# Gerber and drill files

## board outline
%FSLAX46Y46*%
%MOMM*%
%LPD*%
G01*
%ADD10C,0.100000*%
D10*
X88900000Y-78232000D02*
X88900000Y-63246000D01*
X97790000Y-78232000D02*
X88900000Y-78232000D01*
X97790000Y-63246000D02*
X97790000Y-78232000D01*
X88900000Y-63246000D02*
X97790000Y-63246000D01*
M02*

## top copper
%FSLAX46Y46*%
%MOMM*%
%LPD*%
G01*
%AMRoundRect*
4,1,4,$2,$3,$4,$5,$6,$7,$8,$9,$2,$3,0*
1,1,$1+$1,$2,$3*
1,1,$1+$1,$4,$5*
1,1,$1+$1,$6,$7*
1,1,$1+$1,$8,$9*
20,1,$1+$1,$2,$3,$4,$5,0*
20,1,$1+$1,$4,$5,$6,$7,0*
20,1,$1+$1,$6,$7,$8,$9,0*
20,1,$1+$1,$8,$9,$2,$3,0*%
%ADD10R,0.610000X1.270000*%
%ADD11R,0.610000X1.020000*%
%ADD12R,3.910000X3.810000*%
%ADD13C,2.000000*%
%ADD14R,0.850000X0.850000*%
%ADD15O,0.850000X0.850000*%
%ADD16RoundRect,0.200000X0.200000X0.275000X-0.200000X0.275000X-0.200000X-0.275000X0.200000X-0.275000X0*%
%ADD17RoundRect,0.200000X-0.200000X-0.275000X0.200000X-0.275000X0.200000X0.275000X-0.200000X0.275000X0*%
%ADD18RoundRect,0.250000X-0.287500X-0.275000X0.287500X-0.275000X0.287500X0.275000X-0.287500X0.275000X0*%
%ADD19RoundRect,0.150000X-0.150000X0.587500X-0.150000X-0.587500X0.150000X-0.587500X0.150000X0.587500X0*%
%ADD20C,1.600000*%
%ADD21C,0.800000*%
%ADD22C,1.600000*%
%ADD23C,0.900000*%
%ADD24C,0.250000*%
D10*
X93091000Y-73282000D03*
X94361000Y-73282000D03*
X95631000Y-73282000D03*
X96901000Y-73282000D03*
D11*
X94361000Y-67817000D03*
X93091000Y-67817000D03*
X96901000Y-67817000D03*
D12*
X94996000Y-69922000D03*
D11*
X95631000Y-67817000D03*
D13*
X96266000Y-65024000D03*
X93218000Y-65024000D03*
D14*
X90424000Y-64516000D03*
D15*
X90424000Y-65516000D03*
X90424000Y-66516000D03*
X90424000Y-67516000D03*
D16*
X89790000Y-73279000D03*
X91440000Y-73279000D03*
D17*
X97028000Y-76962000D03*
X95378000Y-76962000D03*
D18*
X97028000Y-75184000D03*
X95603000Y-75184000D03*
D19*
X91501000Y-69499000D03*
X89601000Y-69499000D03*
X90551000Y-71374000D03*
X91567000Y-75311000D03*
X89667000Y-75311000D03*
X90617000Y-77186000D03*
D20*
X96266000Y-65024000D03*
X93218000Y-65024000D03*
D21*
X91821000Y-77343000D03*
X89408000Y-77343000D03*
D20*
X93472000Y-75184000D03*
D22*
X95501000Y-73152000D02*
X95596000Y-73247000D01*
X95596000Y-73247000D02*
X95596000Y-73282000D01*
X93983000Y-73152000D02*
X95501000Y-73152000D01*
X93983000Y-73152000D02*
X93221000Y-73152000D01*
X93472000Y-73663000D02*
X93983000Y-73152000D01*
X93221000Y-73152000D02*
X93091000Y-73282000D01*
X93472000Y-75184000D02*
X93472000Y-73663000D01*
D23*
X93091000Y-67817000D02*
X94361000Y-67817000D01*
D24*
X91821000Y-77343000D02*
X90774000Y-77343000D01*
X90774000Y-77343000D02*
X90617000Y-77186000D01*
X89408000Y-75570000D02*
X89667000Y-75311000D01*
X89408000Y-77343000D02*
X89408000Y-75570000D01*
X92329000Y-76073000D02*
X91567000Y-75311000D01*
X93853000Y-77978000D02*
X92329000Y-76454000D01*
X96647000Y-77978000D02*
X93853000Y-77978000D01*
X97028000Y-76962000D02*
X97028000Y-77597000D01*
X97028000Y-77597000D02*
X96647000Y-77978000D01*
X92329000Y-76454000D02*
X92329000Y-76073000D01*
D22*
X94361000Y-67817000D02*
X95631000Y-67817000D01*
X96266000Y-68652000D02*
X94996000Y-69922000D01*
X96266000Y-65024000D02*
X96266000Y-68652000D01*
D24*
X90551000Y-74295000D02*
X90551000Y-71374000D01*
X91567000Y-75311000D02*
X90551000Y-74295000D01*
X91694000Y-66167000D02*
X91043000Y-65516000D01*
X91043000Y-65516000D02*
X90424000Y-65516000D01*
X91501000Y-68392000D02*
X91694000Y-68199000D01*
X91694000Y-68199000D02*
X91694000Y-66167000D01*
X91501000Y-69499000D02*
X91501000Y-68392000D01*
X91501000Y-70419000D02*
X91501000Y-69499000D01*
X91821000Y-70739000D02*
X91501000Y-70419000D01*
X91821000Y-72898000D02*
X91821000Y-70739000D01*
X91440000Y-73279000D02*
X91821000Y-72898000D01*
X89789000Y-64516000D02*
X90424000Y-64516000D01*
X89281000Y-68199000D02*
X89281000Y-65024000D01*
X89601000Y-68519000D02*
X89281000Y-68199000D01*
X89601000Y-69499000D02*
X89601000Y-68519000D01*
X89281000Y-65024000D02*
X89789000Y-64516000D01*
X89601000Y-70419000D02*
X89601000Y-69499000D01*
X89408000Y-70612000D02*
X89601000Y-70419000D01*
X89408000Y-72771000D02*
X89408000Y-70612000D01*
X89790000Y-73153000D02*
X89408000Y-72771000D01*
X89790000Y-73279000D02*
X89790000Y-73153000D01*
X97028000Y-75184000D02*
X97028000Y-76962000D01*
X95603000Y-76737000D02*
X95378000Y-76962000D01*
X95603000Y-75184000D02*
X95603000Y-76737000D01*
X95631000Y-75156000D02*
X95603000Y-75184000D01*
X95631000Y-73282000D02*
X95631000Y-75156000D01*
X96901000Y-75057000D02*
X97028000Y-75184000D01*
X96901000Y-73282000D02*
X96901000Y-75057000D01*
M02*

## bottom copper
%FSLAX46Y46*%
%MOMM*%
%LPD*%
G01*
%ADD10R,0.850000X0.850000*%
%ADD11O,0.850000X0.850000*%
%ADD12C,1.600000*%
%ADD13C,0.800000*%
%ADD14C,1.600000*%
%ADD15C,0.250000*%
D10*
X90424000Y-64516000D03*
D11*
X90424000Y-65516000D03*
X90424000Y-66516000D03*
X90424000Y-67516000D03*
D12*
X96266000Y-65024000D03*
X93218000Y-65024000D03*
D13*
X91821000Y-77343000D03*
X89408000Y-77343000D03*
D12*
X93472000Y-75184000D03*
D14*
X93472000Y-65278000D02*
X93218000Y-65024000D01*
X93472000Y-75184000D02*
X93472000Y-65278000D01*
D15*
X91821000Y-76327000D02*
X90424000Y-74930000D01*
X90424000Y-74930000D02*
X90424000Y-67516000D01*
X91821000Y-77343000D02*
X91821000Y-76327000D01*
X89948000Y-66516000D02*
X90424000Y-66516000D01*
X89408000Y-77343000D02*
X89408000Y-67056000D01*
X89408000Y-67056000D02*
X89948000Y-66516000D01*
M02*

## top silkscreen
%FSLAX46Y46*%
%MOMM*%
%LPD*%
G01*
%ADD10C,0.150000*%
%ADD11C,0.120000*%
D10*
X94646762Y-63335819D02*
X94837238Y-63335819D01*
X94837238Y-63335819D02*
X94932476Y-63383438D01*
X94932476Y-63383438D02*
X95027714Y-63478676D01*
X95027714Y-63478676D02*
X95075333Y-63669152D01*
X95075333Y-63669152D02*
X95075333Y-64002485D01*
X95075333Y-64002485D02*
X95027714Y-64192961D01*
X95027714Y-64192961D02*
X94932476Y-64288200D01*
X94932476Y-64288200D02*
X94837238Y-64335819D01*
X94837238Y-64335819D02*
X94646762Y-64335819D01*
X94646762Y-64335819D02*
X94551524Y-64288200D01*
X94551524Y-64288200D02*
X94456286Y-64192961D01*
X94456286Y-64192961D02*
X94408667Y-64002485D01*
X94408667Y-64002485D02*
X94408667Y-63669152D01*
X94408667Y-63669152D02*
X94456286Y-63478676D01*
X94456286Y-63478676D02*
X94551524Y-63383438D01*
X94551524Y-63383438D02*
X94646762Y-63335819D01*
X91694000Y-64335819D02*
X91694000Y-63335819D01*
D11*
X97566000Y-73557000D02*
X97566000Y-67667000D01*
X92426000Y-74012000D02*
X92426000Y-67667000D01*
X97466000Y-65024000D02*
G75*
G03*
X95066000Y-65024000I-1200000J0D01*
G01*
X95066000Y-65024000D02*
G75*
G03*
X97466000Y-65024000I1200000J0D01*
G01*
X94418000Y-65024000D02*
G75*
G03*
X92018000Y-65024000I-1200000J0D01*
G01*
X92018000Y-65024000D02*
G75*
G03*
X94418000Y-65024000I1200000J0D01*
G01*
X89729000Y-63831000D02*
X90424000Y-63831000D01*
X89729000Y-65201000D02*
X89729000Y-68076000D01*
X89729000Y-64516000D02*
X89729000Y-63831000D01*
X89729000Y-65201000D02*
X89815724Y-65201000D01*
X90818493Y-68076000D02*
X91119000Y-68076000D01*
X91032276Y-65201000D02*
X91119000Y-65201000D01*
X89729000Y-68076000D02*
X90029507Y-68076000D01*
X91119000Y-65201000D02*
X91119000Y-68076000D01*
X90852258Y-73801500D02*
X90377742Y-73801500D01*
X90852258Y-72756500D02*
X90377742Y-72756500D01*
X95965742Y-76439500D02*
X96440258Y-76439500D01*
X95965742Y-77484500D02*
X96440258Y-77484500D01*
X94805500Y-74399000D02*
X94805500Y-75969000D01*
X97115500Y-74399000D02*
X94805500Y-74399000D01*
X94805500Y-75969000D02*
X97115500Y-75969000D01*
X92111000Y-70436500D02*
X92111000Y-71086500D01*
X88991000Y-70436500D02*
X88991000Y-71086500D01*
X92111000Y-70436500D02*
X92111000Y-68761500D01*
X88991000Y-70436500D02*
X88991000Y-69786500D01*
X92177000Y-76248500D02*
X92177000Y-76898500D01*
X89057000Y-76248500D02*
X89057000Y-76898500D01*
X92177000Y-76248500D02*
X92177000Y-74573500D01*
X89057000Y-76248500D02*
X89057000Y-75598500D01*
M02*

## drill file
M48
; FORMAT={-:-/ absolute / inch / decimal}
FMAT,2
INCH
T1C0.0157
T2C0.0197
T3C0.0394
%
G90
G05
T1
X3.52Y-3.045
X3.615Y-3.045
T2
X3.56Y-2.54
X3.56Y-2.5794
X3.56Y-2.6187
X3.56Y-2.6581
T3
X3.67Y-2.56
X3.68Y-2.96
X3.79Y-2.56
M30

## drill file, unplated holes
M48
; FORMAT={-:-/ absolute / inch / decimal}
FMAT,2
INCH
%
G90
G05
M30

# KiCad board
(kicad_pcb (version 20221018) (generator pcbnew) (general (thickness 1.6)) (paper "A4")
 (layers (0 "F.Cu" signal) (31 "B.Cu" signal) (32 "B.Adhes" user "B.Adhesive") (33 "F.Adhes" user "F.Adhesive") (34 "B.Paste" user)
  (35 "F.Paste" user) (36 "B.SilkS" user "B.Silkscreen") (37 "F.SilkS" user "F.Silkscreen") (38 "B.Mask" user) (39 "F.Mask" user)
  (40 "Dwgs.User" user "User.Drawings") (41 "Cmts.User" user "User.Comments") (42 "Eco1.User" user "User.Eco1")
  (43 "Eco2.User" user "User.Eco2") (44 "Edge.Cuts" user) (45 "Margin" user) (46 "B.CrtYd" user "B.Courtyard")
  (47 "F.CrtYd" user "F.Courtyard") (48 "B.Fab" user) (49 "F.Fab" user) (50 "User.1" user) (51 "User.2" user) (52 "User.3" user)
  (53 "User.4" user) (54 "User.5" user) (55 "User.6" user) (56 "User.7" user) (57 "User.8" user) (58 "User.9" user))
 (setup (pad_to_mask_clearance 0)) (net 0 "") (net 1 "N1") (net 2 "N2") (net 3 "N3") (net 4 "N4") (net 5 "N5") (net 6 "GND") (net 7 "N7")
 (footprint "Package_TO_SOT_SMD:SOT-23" (layer "F.Cu") (at 90.617 76.2485 -90)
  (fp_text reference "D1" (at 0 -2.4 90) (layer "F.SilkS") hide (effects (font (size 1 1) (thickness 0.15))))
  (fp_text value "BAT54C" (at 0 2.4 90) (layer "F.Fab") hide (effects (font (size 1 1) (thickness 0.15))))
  (fp_line (start 0 -1.56) (end -1.675 -1.56) (stroke (width 0.12) (type solid)) (layer "F.SilkS"))
  (fp_line (start 0 -1.56) (end 0.65 -1.56) (stroke (width 0.12) (type solid)) (layer "F.SilkS"))
  (fp_line (start 0 1.56) (end -0.65 1.56) (stroke (width 0.12) (type solid)) (layer "F.SilkS"))
  (fp_line (start 0 1.56) (end 0.65 1.56) (stroke (width 0.12) (type solid)) (layer "F.SilkS"))
  (pad "1" smd roundrect (at -0.9375 -0.95 270) (size 1.475 0.6) (layers "F.Cu" "F.Paste" "F.Mask") (roundrect_rratio 0.25) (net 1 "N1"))
  (pad "2" smd roundrect (at -0.9375 0.95 270) (size 1.475 0.6) (layers "F.Cu" "F.Paste" "F.Mask") (roundrect_rratio 0.25) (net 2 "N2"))
  (pad "3" smd roundrect (at 0.9375 0 270) (size 1.475 0.6) (layers "F.Cu" "F.Paste" "F.Mask") (roundrect_rratio 0.25) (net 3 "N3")))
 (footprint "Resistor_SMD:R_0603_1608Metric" (layer "F.Cu") (at 96.203 76.962)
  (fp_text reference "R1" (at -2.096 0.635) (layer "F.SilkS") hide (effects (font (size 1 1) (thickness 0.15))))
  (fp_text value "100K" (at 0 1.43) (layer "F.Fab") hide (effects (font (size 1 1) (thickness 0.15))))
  (fp_line (start -0.237258 -0.5225) (end 0.237258 -0.5225) (stroke (width 0.12) (type solid)) (layer "F.SilkS"))
  (fp_line (start -0.237258 0.5225) (end 0.237258 0.5225) (stroke (width 0.12) (type solid)) (layer "F.SilkS"))
  (pad "1" smd roundrect (at -0.825 0) (size 0.8 0.95) (layers "F.Cu" "F.Paste" "F.Mask") (roundrect_rratio 0.25) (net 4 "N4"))
  (pad "2" smd roundrect (at 0.825 0) (size 0.8 0.95) (layers "F.Cu" "F.Paste" "F.Mask") (roundrect_rratio 0.25) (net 1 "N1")))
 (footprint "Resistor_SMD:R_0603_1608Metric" (layer "F.Cu") (at 90.615 73.279 180)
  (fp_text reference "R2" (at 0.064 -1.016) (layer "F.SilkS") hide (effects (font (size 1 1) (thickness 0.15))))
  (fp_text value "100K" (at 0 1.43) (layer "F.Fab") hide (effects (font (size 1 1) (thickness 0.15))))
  (fp_line (start -0.237258 -0.5225) (end 0.237258 -0.5225) (stroke (width 0.12) (type solid)) (layer "F.SilkS"))
  (fp_line (start -0.237258 0.5225) (end 0.237258 0.5225) (stroke (width 0.12) (type solid)) (layer "F.SilkS"))
  (pad "1" smd roundrect (at -0.825 0 180) (size 0.8 0.95) (layers "F.Cu" "F.Paste" "F.Mask") (roundrect_rratio 0.25) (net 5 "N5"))
  (pad "2" smd roundrect (at 0.825 0 180) (size 0.8 0.95) (layers "F.Cu" "F.Paste" "F.Mask") (roundrect_rratio 0.25) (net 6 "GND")))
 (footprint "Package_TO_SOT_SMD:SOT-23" (layer "F.Cu") (at 90.551 70.4365 -90)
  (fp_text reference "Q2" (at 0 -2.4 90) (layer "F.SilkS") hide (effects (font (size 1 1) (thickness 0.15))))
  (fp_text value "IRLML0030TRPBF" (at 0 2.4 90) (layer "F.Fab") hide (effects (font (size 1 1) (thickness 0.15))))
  (fp_line (start 0 -1.56) (end -1.675 -1.56) (stroke (width 0.12) (type solid)) (layer "F.SilkS"))
  (fp_line (start 0 -1.56) (end 0.65 -1.56) (stroke (width 0.12) (type solid)) (layer "F.SilkS"))
  (fp_line (start 0 1.56) (end -0.65 1.56) (stroke (width 0.12) (type solid)) (layer "F.SilkS"))
  (fp_line (start 0 1.56) (end 0.65 1.56) (stroke (width 0.12) (type solid)) (layer "F.SilkS"))
  (pad "1" smd roundrect (at -0.9375 -0.95 270) (size 1.475 0.6) (layers "F.Cu" "F.Paste" "F.Mask") (roundrect_rratio 0.25) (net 5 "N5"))
  (pad "2" smd roundrect (at -0.9375 0.95 270) (size 1.475 0.6) (layers "F.Cu" "F.Paste" "F.Mask") (roundrect_rratio 0.25) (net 6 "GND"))
  (pad "3" smd roundrect (at 0.9375 0 270) (size 1.475 0.6) (layers "F.Cu" "F.Paste" "F.Mask") (roundrect_rratio 0.25) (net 1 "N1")))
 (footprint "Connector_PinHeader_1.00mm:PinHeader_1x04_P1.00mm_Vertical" (layer "F.Cu") (at 90.424 64.516)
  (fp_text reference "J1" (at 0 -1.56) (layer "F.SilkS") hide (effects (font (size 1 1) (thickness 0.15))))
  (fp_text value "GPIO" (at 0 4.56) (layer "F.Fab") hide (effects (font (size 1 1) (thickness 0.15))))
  (fp_line (start -0.695 -0.685) (end 0 -0.685) (stroke (width 0.12) (type solid)) (layer "F.SilkS"))
  (fp_line (start -0.695 0) (end -0.695 -0.685) (stroke (width 0.12) (type solid)) (layer "F.SilkS"))
  (fp_line (start -0.695 0.685) (end -0.695 3.56) (stroke (width 0.12) (type solid)) (layer "F.SilkS"))
  (fp_line (start -0.695 0.685) (end -0.608276 0.685) (stroke (width 0.12) (type solid)) (layer "F.SilkS"))
  (fp_line (start -0.695 3.56) (end -0.394493 3.56) (stroke (width 0.12) (type solid)) (layer "F.SilkS"))
  (fp_line (start 0.394493 3.56) (end 0.695 3.56) (stroke (width 0.12) (type solid)) (layer "F.SilkS"))
  (fp_line (start 0.608276 0.685) (end 0.695 0.685) (stroke (width 0.12) (type solid)) (layer "F.SilkS"))
  (fp_line (start 0.695 0.685) (end 0.695 3.56) (stroke (width 0.12) (type solid)) (layer "F.SilkS"))
  (pad "1" thru_hole rect (at 0 0) (size 0.85 0.85) (drill 0.5) (layers "*.Cu" "*.Mask") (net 6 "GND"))
  (pad "2" thru_hole oval (at 0 1) (size 0.85 0.85) (drill 0.5) (layers "*.Cu" "*.Mask") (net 5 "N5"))
  (pad "3" thru_hole oval (at 0 2) (size 0.85 0.85) (drill 0.5) (layers "*.Cu" "*.Mask") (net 2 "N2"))
  (pad "4" thru_hole oval (at 0 3) (size 0.85 0.85) (drill 0.5) (layers "*.Cu" "*.Mask") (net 3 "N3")))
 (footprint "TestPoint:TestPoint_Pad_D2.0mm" (layer "F.Cu") (at 96.266 65.024)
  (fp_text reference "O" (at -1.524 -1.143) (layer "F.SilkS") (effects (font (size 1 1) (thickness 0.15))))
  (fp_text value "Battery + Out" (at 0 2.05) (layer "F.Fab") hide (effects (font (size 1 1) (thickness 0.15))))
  (fp_circle (center 0 0) (end 0 1.2) (stroke (width 0.12) (type solid)) (fill none) (layer "F.SilkS"))
  (pad "1" smd circle (at 0 0) (size 2 2) (layers "F.Cu" "F.Mask") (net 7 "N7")))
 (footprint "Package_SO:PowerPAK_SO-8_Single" (layer "F.Cu") (at 94.996 70.612 90)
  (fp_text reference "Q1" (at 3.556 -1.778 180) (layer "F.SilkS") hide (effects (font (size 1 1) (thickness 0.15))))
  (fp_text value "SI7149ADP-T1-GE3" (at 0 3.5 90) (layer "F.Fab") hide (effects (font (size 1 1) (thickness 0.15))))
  (fp_line (start -3.4 -2.57) (end 2.945 -2.57) (stroke (width 0.12) (type solid)) (layer "F.SilkS"))
  (fp_line (start -2.945 2.57) (end 2.945 2.57) (stroke (width 0.12) (type solid)) (layer "F.SilkS"))
  (pad "1" smd rect (at -2.67 -1.905 90) (size 1.27 0.61) (layers "F.Cu" "F.Paste" "F.Mask") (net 4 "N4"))
  (pad "2" smd rect (at -2.67 -0.635 90) (size 1.27 0.61) (layers "F.Cu" "F.Paste" "F.Mask") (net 4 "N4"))
  (pad "3" smd rect (at -2.67 0.635 90) (size 1.27 0.61) (layers "F.Cu" "F.Paste" "F.Mask") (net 4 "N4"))
  (pad "4" smd rect (at -2.67 1.905 90) (size 1.27 0.61) (layers "F.Cu" "F.Paste" "F.Mask") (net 1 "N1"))
  (pad "5" smd rect (at 0.69 0 90) (size 3.81 3.91) (layers "F.Cu" "F.Paste" "F.Mask") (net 7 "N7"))
  (pad "5" smd rect (at 2.795 -1.905 90) (size 1.02 0.61) (layers "F.Cu" "F.Paste" "F.Mask") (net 7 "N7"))
  (pad "5" smd rect (at 2.795 -0.635 90) (size 1.02 0.61) (layers "F.Cu" "F.Paste" "F.Mask") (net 7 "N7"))
  (pad "5" smd rect (at 2.795 0.635 90) (size 1.02 0.61) (layers "F.Cu" "F.Paste" "F.Mask") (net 7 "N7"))
  (pad "5" smd rect (at 2.795 1.905 90) (size 1.02 0.61) (layers "F.Cu" "F.Paste" "F.Mask") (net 7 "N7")))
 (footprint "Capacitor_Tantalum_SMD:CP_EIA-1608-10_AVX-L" (layer "F.Cu") (at 96.3155 75.184)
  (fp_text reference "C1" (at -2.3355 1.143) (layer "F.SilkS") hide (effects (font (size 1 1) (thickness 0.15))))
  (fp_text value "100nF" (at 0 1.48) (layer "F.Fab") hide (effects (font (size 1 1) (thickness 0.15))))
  (fp_line (start -1.51 -0.785) (end -1.51 0.785) (stroke (width 0.12) (type solid)) (layer "F.SilkS"))
  (fp_line (start -1.51 0.785) (end 0.8 0.785) (stroke (width 0.12) (type solid)) (layer "F.SilkS"))
  (fp_line (start 0.8 -0.785) (end -1.51 -0.785) (stroke (width 0.12) (type solid)) (layer "F.SilkS"))
  (pad "1" smd roundrect (at -0.7125 0) (size 1.075 1.05) (layers "F.Cu" "F.Paste" "F.Mask") (roundrect_rratio 0.2380952381) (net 4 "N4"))
  (pad "2" smd roundrect (at 0.7125 0) (size 1.075 1.05) (layers "F.Cu" "F.Paste" "F.Mask") (roundrect_rratio 0.2380952381) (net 1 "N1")))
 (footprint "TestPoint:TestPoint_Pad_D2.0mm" (layer "F.Cu") (at 93.218 65.024)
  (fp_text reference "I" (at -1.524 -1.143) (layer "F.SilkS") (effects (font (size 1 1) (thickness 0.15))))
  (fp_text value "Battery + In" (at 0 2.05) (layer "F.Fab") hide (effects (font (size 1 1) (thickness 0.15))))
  (fp_circle (center 0 0) (end 0 1.2) (stroke (width 0.12) (type solid)) (fill none) (layer "F.SilkS"))
  (pad "1" smd circle (at 0 0) (size 2 2) (layers "F.Cu" "F.Mask") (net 4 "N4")))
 (gr_line (start 97.79 63.246) (end 97.79 78.232) (stroke (width 0.1) (type default)) (layer "Edge.Cuts"))
 (gr_line (start 88.9 63.246) (end 97.79 63.246) (stroke (width 0.1) (type default)) (layer "Edge.Cuts"))
 (gr_line (start 88.9 78.232) (end 88.9 63.246) (stroke (width 0.1) (type default)) (layer "Edge.Cuts"))
 (gr_line (start 97.79 78.232) (end 88.9 78.232) (stroke (width 0.1) (type default)) (layer "Edge.Cuts"))
 (segment (start 91.501 70.419) (end 91.501 69.499) (width 0.25) (layer "F.Cu") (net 5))
 (segment (start 91.694 68.199) (end 91.694 66.167) (width 0.25) (layer "F.Cu") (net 5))
 (segment (start 91.043 65.516) (end 90.424 65.516) (width 0.25) (layer "F.Cu") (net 5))
 (segment (start 91.501 68.392) (end 91.694 68.199) (width 0.25) (layer "F.Cu") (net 5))
 (segment (start 91.694 66.167) (end 91.043 65.516) (width 0.25) (layer "F.Cu") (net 5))
 (segment (start 91.44 73.279) (end 91.821 72.898) (width 0.25) (layer "F.Cu") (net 5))
 (segment (start 91.821 70.739) (end 91.501 70.419) (width 0.25) (layer "F.Cu") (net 5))
 (segment (start 91.821 72.898) (end 91.821 70.739) (width 0.25) (layer "F.Cu") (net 5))
 (segment (start 91.501 69.499) (end 91.501 68.392) (width 0.25) (layer "F.Cu") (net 5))
 (segment (start 89.408 77.343) (end 89.408 75.57) (width 0.25) (layer "F.Cu") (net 2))
 (segment (start 89.408 75.57) (end 89.667 75.311) (width 0.25) (layer "F.Cu") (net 2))
 (via (at 89.408 77.343) (size 0.8) (drill 0.4) (layers "F.Cu" "B.Cu") (free) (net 2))
 (segment (start 89.408 77.343) (end 89.408 67.056) (width 0.25) (layer "B.Cu") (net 2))
 (segment (start 89.408 67.056) (end 89.948 66.516) (width 0.25) (layer "B.Cu") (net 2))
 (segment (start 89.948 66.516) (end 90.424 66.516) (width 0.25) (layer "B.Cu") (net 2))
 (segment (start 97.028 75.184) (end 97.028 76.962) (width 0.25) (layer "F.Cu") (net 1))
 (segment (start 92.329 76.073) (end 91.567 75.311) (width 0.25) (layer "F.Cu") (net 1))
 (segment (start 97.028 76.962) (end 97.028 77.597) (width 0.25) (layer "F.Cu") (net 1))
 (segment (start 91.567 75.311) (end 90.551 74.295) (width 0.25) (layer "F.Cu") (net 1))
 (segment (start 96.901 75.057) (end 97.028 75.184) (width 0.25) (layer "F.Cu") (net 1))
 (segment (start 96.901 73.282) (end 96.901 75.057) (width 0.25) (layer "F.Cu") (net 1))
 (segment (start 92.329 76.454) (end 92.329 76.073) (width 0.25) (layer "F.Cu") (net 1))
 (segment (start 96.647 77.978) (end 93.853 77.978) (width 0.25) (layer "F.Cu") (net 1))
 (segment (start 90.551 74.295) (end 90.551 71.374) (width 0.25) (layer "F.Cu") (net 1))
 (segment (start 93.853 77.978) (end 92.329 76.454) (width 0.25) (layer "F.Cu") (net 1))
 (segment (start 97.028 77.597) (end 96.647 77.978) (width 0.25) (layer "F.Cu") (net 1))
 (segment (start 93.472 73.663) (end 93.983 73.152) (width 1.6) (layer "F.Cu") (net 4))
 (segment (start 95.603 76.737) (end 95.378 76.962) (width 0.25) (layer "F.Cu") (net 4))
 (segment (start 95.596 73.247) (end 95.596 73.282) (width 1.6) (layer "F.Cu") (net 4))
 (segment (start 93.221 73.152) (end 93.091 73.282) (width 1.6) (layer "F.Cu") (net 4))
 (segment (start 95.603 75.184) (end 95.603 76.737) (width 0.25) (layer "F.Cu") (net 4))
 (segment (start 93.983 73.152) (end 95.501 73.152) (width 1.6) (layer "F.Cu") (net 4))
 (segment (start 95.501 73.152) (end 95.596 73.247) (width 1.6) (layer "F.Cu") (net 4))
 (segment (start 93.472 75.184) (end 93.472 73.663) (width 1.6) (layer "F.Cu") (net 4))
 (segment (start 95.631 75.156) (end 95.603 75.184) (width 0.25) (layer "F.Cu") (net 4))
 (segment (start 95.631 73.282) (end 95.631 75.156) (width 0.25) (layer "F.Cu") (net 4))
 (segment (start 93.983 73.152) (end 93.221 73.152) (width 1.6) (layer "F.Cu") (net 4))
 (via (at 93.218 65.024) (size 1.6) (drill 1) (layers "F.Cu" "B.Cu") (free) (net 4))
 (via (at 93.472 75.184) (size 1.6) (drill 1) (layers "F.Cu" "B.Cu") (free) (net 4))
 (segment (start 93.472 75.184) (end 93.472 65.278) (width 1.6) (layer "B.Cu") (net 4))
 (segment (start 93.472 65.278) (end 93.218 65.024) (width 1.6) (layer "B.Cu") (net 4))
 (segment (start 96.266 68.652) (end 94.996 69.922) (width 1.6) (layer "F.Cu") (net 7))
 (segment (start 93.091 67.817) (end 94.361 67.817) (width 0.9) (layer "F.Cu") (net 7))
 (segment (start 94.361 67.817) (end 95.631 67.817) (width 1.6) (layer "F.Cu") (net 7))
 (segment (start 96.266 65.024) (end 96.266 68.652) (width 1.6) (layer "F.Cu") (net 7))
 (via (at 96.266 65.024) (size 1.6) (drill 1) (layers "F.Cu" "B.Cu") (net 7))
 (segment (start 89.79 73.153) (end 89.408 72.771) (width 0.25) (layer "F.Cu") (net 6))
 (segment (start 89.281 65.024) (end 89.789 64.516) (width 0.25) (layer "F.Cu") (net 6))
 (segment (start 89.79 73.279) (end 89.79 73.153) (width 0.25) (layer "F.Cu") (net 6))
 (segment (start 89.601 69.499) (end 89.601 68.519) (width 0.25) (layer "F.Cu") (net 6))
 (segment (start 89.408 70.612) (end 89.601 70.419) (width 0.25) (layer "F.Cu") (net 6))
 (segment (start 89.601 70.419) (end 89.601 69.499) (width 0.25) (layer "F.Cu") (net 6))
 (segment (start 89.601 68.519) (end 89.281 68.199) (width 0.25) (layer "F.Cu") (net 6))
 (segment (start 89.408 72.771) (end 89.408 70.612) (width 0.25) (layer "F.Cu") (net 6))
 (segment (start 89.281 68.199) (end 89.281 65.024) (width 0.25) (layer "F.Cu") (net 6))
 (segment (start 89.789 64.516) (end 90.424 64.516) (width 0.25) (layer "F.Cu") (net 6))
 (segment (start 91.821 77.343) (end 90.774 77.343) (width 0.25) (layer "F.Cu") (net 3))
 (segment (start 90.774 77.343) (end 90.617 77.186) (width 0.25) (layer "F.Cu") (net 3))
 (via (at 91.821 77.343) (size 0.8) (drill 0.4) (layers "F.Cu" "B.Cu") (free) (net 3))
 (segment (start 91.821 76.327) (end 90.424 74.93) (width 0.25) (layer "B.Cu") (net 3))
 (segment (start 91.821 77.343) (end 91.821 76.327) (width 0.25) (layer "B.Cu") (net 3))
 (segment (start 90.424 74.93) (end 90.424 67.516) (width 0.25) (layer "B.Cu") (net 3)))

